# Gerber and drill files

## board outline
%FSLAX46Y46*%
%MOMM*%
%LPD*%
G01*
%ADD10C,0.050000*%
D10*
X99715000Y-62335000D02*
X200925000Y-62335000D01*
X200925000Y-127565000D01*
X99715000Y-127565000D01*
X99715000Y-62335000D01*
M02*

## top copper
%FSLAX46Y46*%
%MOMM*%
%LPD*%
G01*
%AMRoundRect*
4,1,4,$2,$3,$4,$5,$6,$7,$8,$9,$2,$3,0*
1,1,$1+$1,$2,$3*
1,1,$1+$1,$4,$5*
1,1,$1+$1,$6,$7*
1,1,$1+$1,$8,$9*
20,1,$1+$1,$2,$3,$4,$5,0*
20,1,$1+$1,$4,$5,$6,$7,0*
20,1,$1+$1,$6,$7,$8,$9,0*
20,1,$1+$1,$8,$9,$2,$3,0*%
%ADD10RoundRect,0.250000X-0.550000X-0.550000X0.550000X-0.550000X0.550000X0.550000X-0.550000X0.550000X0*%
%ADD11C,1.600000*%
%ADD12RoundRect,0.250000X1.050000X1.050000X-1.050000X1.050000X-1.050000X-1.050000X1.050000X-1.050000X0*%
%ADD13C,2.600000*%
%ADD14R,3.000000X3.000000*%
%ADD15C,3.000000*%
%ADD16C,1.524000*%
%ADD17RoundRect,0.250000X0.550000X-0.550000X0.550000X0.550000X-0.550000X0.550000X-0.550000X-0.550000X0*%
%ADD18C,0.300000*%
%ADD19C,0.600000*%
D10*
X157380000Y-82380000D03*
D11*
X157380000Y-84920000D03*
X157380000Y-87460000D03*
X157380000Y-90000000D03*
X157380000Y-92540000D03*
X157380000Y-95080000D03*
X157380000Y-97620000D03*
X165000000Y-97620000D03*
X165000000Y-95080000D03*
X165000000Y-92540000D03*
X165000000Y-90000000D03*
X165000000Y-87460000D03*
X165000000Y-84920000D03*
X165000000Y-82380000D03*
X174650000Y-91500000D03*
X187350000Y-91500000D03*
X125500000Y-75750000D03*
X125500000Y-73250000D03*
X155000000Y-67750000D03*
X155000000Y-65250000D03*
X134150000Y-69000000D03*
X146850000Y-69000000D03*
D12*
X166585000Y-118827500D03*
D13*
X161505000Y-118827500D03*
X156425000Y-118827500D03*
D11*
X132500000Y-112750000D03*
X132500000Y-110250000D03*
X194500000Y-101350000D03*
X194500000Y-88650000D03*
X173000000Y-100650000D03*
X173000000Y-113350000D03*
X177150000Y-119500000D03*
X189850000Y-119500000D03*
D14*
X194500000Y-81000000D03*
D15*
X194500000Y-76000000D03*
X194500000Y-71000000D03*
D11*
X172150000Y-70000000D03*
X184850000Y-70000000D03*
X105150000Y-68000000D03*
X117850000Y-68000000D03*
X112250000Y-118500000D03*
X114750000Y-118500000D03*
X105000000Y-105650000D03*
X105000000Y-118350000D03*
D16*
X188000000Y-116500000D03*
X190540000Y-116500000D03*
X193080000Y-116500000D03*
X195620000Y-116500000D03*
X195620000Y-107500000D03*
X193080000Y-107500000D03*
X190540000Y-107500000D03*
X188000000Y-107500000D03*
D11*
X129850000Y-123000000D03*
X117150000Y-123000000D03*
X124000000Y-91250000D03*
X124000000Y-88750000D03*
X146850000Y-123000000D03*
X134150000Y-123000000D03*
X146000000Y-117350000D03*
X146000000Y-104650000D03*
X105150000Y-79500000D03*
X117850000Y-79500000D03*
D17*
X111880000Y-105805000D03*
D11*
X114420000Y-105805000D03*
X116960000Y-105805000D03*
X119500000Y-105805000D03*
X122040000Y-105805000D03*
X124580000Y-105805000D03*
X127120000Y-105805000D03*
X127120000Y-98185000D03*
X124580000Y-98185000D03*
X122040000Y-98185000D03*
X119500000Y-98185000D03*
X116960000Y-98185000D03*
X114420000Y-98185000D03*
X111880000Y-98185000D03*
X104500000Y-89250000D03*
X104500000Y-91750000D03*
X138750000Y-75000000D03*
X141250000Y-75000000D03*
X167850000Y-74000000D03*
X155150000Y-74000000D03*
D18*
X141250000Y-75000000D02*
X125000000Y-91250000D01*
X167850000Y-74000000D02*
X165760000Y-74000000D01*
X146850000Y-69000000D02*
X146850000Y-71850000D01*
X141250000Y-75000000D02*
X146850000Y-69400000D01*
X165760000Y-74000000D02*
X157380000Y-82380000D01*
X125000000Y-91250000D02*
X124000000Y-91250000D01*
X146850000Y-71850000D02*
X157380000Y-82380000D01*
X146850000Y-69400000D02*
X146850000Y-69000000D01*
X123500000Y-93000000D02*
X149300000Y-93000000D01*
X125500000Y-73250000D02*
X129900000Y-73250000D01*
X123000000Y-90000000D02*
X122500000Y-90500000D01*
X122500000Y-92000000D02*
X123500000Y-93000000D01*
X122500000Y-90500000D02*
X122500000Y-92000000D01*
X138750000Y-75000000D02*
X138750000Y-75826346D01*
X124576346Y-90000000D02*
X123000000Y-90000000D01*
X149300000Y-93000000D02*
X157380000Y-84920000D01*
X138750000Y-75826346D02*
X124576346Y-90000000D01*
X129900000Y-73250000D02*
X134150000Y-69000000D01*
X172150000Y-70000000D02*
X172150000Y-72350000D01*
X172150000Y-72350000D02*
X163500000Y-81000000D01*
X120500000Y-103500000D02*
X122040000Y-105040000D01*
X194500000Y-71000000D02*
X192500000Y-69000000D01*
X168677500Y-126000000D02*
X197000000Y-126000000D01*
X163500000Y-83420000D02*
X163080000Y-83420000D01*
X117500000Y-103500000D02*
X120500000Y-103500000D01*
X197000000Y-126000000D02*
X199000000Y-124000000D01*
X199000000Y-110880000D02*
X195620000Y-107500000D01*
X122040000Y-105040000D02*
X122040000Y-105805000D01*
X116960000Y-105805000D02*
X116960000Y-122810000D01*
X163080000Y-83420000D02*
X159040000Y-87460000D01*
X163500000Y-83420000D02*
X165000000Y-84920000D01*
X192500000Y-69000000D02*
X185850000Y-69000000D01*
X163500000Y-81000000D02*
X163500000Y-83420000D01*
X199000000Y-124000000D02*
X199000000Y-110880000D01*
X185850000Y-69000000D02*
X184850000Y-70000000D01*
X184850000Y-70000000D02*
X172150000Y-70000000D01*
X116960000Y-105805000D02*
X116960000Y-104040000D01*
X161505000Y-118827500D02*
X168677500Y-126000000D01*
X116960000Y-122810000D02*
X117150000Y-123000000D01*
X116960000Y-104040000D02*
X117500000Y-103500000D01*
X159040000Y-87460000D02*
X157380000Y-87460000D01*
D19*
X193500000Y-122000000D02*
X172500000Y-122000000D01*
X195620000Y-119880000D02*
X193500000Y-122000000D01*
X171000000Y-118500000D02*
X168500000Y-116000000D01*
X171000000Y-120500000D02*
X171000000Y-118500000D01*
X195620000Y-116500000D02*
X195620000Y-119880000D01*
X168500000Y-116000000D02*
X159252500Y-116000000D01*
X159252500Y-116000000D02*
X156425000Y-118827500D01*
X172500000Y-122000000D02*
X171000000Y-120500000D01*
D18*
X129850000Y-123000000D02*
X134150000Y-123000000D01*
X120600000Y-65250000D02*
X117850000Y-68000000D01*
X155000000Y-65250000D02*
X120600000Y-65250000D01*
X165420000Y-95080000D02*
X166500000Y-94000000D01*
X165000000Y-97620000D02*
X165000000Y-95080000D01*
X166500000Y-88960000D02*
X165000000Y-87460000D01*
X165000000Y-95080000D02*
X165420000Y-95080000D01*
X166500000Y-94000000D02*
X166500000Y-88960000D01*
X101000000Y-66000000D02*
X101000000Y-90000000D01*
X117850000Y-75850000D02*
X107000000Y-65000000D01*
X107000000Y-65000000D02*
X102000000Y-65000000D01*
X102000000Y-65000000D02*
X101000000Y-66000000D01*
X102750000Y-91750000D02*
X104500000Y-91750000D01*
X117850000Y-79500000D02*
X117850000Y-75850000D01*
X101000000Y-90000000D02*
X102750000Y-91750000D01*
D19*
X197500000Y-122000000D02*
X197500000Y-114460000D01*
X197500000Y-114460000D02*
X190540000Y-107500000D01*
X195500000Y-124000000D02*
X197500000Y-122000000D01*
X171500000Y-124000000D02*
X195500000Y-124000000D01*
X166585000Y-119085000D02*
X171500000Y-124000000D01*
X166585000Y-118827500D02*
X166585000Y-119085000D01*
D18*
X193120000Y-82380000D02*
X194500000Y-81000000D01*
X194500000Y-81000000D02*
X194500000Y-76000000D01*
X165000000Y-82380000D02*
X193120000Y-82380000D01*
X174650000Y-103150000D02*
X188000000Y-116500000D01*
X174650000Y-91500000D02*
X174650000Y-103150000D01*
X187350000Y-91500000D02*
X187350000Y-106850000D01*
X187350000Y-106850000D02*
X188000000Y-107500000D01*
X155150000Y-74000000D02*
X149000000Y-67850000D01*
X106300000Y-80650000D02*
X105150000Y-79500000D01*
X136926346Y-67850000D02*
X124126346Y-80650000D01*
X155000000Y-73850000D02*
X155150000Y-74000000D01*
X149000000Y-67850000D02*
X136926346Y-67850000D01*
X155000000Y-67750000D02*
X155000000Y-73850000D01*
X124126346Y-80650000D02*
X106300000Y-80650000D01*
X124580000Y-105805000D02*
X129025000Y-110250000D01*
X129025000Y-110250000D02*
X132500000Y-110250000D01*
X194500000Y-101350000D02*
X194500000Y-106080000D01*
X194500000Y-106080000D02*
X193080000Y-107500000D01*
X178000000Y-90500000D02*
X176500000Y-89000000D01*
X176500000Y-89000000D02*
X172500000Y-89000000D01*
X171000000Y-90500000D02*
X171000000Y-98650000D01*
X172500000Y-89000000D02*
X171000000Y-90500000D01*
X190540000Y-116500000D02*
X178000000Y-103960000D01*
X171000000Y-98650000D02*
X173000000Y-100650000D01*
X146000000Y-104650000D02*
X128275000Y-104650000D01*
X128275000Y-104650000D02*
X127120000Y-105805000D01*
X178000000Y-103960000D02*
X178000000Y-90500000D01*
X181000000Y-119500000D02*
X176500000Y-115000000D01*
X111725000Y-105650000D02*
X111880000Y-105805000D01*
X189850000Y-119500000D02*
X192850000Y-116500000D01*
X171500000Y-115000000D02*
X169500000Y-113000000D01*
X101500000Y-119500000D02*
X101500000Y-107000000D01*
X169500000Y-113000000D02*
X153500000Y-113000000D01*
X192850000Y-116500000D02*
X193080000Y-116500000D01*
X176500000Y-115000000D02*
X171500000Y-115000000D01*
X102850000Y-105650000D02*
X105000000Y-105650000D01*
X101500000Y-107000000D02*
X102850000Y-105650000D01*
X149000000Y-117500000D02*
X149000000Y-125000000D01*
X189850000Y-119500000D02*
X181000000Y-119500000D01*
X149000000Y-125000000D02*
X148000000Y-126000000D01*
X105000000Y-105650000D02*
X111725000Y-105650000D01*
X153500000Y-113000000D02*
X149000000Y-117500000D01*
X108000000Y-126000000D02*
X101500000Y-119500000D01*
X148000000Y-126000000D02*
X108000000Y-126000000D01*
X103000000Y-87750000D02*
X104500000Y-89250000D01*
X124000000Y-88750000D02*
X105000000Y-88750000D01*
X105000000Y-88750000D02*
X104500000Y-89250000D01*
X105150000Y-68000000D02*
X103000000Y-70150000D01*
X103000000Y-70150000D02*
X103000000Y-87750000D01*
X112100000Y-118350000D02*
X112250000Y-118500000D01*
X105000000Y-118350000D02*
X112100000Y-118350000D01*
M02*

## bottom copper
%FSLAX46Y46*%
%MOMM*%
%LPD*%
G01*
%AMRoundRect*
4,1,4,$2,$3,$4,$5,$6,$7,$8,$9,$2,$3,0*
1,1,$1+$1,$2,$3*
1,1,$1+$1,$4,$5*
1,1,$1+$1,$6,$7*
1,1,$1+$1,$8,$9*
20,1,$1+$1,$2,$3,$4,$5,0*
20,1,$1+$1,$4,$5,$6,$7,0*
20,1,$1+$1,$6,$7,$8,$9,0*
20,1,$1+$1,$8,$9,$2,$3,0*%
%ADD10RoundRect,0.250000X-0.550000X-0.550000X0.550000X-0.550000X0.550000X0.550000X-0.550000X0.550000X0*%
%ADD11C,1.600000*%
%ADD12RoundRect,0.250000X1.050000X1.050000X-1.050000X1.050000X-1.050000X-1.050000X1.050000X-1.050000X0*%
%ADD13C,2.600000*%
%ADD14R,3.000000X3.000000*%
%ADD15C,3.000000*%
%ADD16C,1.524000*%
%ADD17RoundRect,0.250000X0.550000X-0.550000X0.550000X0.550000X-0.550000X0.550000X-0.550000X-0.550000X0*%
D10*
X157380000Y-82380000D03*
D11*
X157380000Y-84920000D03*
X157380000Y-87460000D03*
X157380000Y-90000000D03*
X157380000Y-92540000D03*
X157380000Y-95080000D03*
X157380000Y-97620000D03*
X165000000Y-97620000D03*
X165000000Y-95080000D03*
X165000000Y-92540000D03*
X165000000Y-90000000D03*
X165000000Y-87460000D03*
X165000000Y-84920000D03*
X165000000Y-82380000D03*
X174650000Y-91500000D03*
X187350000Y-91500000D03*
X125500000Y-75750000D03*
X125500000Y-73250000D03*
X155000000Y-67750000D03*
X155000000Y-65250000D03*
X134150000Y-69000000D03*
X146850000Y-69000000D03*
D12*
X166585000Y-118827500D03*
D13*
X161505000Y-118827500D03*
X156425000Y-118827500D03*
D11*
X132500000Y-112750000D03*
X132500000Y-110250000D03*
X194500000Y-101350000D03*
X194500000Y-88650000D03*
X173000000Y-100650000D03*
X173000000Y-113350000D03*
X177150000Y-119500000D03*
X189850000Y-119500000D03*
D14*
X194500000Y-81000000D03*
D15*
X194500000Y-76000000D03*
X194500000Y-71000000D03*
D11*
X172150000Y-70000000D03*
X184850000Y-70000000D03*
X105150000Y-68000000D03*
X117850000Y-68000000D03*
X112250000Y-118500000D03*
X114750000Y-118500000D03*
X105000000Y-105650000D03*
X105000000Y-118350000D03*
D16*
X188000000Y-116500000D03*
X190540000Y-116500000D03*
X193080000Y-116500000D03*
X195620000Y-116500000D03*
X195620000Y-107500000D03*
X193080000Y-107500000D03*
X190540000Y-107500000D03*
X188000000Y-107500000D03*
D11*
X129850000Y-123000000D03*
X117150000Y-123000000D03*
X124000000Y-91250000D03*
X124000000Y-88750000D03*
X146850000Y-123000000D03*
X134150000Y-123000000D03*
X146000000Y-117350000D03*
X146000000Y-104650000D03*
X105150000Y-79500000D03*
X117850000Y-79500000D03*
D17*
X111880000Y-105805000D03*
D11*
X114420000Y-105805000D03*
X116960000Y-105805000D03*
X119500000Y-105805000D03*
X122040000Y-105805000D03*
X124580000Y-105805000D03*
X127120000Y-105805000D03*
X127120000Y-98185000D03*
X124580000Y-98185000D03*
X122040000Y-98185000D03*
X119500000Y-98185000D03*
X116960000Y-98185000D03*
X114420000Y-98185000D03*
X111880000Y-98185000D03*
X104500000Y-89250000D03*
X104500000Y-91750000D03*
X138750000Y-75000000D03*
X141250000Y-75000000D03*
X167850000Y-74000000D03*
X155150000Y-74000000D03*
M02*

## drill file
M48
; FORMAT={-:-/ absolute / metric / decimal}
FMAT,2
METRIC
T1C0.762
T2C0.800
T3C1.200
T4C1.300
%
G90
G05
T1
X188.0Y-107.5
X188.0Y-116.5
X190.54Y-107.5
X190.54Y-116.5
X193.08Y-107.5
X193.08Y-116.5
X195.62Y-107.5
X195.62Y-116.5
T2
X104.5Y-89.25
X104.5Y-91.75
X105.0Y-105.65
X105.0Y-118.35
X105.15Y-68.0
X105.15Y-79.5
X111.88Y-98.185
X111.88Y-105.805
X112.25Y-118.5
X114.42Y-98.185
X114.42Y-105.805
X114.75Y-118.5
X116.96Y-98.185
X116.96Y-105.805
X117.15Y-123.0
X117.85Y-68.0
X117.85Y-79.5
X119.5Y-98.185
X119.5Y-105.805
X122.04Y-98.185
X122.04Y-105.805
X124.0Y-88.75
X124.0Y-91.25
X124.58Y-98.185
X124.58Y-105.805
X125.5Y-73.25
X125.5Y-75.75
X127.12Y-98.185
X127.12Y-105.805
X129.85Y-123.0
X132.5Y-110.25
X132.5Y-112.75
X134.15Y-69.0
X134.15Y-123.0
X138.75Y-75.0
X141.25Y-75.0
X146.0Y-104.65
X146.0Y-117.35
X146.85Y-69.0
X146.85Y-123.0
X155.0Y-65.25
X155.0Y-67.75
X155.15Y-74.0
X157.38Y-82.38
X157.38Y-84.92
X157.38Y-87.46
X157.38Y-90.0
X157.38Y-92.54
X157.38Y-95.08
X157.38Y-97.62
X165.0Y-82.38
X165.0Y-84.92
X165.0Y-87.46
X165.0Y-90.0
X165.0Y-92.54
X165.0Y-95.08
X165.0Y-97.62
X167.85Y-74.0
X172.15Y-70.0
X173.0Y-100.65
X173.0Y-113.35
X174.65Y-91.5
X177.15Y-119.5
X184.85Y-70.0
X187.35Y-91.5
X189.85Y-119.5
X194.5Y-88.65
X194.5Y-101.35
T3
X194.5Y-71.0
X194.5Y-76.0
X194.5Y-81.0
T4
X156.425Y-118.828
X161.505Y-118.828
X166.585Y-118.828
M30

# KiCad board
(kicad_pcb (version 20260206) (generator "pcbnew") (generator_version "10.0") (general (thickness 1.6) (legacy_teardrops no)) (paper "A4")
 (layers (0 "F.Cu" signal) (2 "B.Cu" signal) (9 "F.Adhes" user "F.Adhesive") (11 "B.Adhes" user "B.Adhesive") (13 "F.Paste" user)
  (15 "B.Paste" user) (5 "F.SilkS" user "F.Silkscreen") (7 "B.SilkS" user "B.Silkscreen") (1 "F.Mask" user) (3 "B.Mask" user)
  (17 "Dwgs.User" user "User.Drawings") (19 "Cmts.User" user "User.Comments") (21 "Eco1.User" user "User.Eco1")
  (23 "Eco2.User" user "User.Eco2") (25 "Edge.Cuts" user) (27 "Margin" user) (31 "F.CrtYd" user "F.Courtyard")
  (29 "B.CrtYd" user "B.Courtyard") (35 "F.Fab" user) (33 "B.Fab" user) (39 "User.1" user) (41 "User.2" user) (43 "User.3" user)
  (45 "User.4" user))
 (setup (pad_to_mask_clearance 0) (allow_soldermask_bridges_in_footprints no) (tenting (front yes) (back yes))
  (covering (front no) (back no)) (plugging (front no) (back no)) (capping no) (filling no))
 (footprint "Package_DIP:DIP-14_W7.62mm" (layer "F.Cu") (at 157.38 82.38)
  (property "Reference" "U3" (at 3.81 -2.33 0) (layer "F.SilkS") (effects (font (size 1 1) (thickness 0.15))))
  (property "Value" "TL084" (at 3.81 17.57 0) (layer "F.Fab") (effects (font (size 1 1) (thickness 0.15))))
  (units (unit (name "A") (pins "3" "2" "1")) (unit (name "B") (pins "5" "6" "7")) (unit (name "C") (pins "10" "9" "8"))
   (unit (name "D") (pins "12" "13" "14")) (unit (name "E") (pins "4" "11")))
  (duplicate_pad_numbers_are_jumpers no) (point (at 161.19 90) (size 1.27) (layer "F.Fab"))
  (pad "1" thru_hole roundrect (at 0 0) (size 1.6 1.6) (drill 0.8) (layers "*.Cu" "*.Mask") (remove_unused_layers no)
   (roundrect_rratio 0.15625) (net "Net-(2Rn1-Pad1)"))
  (pad "2" thru_hole circle (at 0 2.54) (size 1.6 1.6) (drill 0.8) (layers "*.Cu" "*.Mask") (remove_unused_layers no) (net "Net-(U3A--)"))
  (pad "3" thru_hole circle (at 0 5.08) (size 1.6 1.6) (drill 0.8) (layers "*.Cu" "*.Mask") (remove_unused_layers no) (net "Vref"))
  (pad "4" thru_hole circle (at 0 7.62) (size 1.6 1.6) (drill 0.8) (layers "*.Cu" "*.Mask") (remove_unused_layers no) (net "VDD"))
  (pad "5" thru_hole circle (at 0 10.16) (size 1.6 1.6) (drill 0.8) (layers "*.Cu" "*.Mask") (remove_unused_layers no) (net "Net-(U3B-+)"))
  (pad "6" thru_hole circle (at 0 12.7) (size 1.6 1.6) (drill 0.8) (layers "*.Cu" "*.Mask") (remove_unused_layers no) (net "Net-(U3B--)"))
  (pad "7" thru_hole circle (at 0 15.24) (size 1.6 1.6) (drill 0.8) (layers "*.Cu" "*.Mask") (remove_unused_layers no) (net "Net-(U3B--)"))
  (pad "8" thru_hole circle (at 7.62 15.24) (size 1.6 1.6) (drill 0.8) (layers "*.Cu" "*.Mask") (remove_unused_layers no)
   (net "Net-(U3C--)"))
  (pad "9" thru_hole circle (at 7.62 12.7) (size 1.6 1.6) (drill 0.8) (layers "*.Cu" "*.Mask") (remove_unused_layers no) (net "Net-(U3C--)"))
  (pad "10" thru_hole circle (at 7.62 10.16) (size 1.6 1.6) (drill 0.8) (layers "*.Cu" "*.Mask") (remove_unused_layers no)
   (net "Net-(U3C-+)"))
  (pad "11" thru_hole circle (at 7.62 7.62) (size 1.6 1.6) (drill 0.8) (layers "*.Cu" "*.Mask") (remove_unused_layers no) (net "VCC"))
  (pad "12" thru_hole circle (at 7.62 5.08) (size 1.6 1.6) (drill 0.8) (layers "*.Cu" "*.Mask") (remove_unused_layers no)
   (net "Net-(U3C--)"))
  (pad "13" thru_hole circle (at 7.62 2.54) (size 1.6 1.6) (drill 0.8) (layers "*.Cu" "*.Mask") (remove_unused_layers no) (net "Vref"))
  (pad "14" thru_hole circle (at 7.62 0) (size 1.6 1.6) (drill 0.8) (layers "*.Cu" "*.Mask") (remove_unused_layers no) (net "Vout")))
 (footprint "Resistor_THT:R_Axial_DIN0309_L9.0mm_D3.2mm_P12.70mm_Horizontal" (layer "F.Cu") (at 174.65 91.5)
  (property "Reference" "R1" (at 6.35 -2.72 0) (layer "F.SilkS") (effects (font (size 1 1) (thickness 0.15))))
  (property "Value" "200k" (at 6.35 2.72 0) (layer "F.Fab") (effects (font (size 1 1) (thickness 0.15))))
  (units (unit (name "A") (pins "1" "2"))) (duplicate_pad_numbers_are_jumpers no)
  (pad "1" thru_hole circle (at 0 0) (size 1.6 1.6) (drill 0.8) (layers "*.Cu" "*.Mask") (remove_unused_layers no) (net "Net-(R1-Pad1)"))
  (pad "2" thru_hole circle (at 12.7 0) (size 1.6 1.6) (drill 0.8) (layers "*.Cu" "*.Mask") (remove_unused_layers no) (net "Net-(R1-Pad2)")))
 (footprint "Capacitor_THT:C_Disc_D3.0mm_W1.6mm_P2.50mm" (layer "F.Cu") (at 125.5 75.75 90)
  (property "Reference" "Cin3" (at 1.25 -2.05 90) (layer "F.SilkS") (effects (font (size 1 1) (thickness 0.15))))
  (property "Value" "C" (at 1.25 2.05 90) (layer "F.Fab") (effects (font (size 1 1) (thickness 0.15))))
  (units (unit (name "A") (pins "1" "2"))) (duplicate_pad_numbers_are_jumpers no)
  (pad "1" thru_hole circle (at 0 0 90) (size 1.6 1.6) (drill 0.8) (layers "*.Cu" "*.Mask") (remove_unused_layers no)
   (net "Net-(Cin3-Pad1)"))
  (pad "2" thru_hole circle (at 2.5 0 90) (size 1.6 1.6) (drill 0.8) (layers "*.Cu" "*.Mask") (remove_unused_layers no) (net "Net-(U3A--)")))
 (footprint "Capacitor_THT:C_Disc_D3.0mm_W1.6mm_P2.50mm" (layer "F.Cu") (at 155 67.75 90)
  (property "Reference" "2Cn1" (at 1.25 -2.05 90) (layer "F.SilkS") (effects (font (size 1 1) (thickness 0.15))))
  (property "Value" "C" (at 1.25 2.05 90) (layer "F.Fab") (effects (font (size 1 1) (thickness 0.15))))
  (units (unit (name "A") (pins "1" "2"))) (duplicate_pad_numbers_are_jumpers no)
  (pad "1" thru_hole circle (at 0 0 90) (size 1.6 1.6) (drill 0.8) (layers "*.Cu" "*.Mask") (remove_unused_layers no)
   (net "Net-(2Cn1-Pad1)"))
  (pad "2" thru_hole circle (at 2.5 0 90) (size 1.6 1.6) (drill 0.8) (layers "*.Cu" "*.Mask") (remove_unused_layers no) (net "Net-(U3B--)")))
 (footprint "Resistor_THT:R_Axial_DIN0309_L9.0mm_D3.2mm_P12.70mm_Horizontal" (layer "F.Cu") (at 134.15 69)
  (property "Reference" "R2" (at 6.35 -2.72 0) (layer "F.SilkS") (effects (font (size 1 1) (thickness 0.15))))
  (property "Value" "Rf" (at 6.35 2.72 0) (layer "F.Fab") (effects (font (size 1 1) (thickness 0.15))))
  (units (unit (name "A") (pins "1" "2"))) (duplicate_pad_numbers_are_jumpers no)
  (pad "1" thru_hole circle (at 0 0) (size 1.6 1.6) (drill 0.8) (layers "*.Cu" "*.Mask") (remove_unused_layers no) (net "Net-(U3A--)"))
  (pad "2" thru_hole circle (at 12.7 0) (size 1.6 1.6) (drill 0.8) (layers "*.Cu" "*.Mask") (remove_unused_layers no)
   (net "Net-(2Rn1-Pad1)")))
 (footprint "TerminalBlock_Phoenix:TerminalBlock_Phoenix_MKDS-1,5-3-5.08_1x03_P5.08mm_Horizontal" (layer "F.Cu") (at 166.585 118.8275 180)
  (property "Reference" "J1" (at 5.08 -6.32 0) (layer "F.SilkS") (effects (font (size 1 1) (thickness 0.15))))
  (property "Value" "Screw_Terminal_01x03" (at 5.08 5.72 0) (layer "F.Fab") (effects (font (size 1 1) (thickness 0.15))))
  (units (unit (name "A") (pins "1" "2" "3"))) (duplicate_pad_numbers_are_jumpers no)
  (pad "1" thru_hole roundrect (at 0 0 180) (size 2.6 2.6) (drill 1.3) (layers "*.Cu" "*.Mask") (remove_unused_layers no)
   (roundrect_rratio 0.096154) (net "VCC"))
  (pad "2" thru_hole circle (at 5.08 0 180) (size 2.6 2.6) (drill 1.3) (layers "*.Cu" "*.Mask") (remove_unused_layers no) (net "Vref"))
  (pad "3" thru_hole circle (at 10.16 0 180) (size 2.6 2.6) (drill 1.3) (layers "*.Cu" "*.Mask") (remove_unused_layers no) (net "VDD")))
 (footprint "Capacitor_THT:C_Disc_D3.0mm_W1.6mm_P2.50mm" (layer "F.Cu") (at 132.5 112.75 90)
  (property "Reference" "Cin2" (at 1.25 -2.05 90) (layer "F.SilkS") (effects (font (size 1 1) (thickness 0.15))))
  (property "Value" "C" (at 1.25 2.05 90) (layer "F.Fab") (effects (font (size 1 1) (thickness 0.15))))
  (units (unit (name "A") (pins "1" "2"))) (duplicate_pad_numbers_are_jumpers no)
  (pad "1" thru_hole circle (at 0 0 90) (size 1.6 1.6) (drill 0.8) (layers "*.Cu" "*.Mask") (remove_unused_layers no)
   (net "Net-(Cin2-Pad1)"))
  (pad "2" thru_hole circle (at 2.5 0 90) (size 1.6 1.6) (drill 0.8) (layers "*.Cu" "*.Mask") (remove_unused_layers no) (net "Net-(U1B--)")))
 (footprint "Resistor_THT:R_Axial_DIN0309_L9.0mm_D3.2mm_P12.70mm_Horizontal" (layer "F.Cu") (at 194.5 101.35 90)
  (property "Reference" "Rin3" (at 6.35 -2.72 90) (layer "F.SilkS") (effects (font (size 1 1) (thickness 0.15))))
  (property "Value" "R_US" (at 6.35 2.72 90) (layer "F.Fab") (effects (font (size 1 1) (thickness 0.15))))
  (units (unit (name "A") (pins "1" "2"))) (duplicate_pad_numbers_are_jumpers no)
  (pad "1" thru_hole circle (at 0 0 90) (size 1.6 1.6) (drill 0.8) (layers "*.Cu" "*.Mask") (remove_unused_layers no) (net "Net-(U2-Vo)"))
  (pad "2" thru_hole circle (at 12.7 0 90) (size 1.6 1.6) (drill 0.8) (layers "*.Cu" "*.Mask") (remove_unused_layers no)
   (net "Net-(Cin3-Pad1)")))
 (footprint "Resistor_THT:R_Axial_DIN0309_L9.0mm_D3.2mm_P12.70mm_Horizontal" (layer "F.Cu") (at 173 100.65 -90)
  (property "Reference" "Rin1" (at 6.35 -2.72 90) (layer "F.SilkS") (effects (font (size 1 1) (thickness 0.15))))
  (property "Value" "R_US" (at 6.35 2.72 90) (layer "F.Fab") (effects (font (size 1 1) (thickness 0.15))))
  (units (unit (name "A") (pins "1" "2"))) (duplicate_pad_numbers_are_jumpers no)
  (pad "1" thru_hole circle (at 0 0 270) (size 1.6 1.6) (drill 0.8) (layers "*.Cu" "*.Mask") (remove_unused_layers no) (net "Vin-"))
  (pad "2" thru_hole circle (at 12.7 0 270) (size 1.6 1.6) (drill 0.8) (layers "*.Cu" "*.Mask") (remove_unused_layers no)
   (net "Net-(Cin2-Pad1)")))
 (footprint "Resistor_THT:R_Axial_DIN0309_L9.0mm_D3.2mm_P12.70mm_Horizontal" (layer "F.Cu") (at 177.15 119.5)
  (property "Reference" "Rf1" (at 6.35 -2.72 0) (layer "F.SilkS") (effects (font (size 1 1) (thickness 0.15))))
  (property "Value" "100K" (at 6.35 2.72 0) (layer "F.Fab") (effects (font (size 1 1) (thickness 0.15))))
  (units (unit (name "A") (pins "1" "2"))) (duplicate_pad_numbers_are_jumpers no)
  (pad "1" thru_hole circle (at 0 0) (size 1.6 1.6) (drill 0.8) (layers "*.Cu" "*.Mask") (remove_unused_layers no) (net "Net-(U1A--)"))
  (pad "2" thru_hole circle (at 12.7 0) (size 1.6 1.6) (drill 0.8) (layers "*.Cu" "*.Mask") (remove_unused_layers no) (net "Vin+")))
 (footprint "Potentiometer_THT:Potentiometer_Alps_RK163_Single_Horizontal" (layer "F.Cu") (at 194.5 81 180)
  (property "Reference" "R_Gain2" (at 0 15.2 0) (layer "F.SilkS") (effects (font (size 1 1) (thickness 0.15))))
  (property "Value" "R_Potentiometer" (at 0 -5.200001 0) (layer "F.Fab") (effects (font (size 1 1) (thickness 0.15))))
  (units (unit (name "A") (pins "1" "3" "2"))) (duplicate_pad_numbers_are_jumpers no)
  (pad "1" thru_hole rect (at 0 0) (size 3 3) (drill 1.2) (layers "*.Cu" "*.Mask") (remove_unused_layers no) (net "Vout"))
  (pad "2" thru_hole circle (at 0 5) (size 3 3) (drill 1.2) (layers "*.Cu" "*.Mask") (remove_unused_layers no) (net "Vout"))
  (pad "3" thru_hole circle (at 0 10) (size 3 3) (drill 1.2) (layers "*.Cu" "*.Mask") (remove_unused_layers no) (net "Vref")))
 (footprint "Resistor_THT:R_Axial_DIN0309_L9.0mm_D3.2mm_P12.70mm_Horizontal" (layer "F.Cu") (at 172.15 70)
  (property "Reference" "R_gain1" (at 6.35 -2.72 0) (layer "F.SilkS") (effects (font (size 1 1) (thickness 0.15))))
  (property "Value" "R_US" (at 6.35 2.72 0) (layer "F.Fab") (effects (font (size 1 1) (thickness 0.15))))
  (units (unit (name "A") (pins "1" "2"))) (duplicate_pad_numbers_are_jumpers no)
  (pad "1" thru_hole circle (at 0 0) (size 1.6 1.6) (drill 0.8) (layers "*.Cu" "*.Mask") (remove_unused_layers no) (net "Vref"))
  (pad "2" thru_hole circle (at 12.7 0) (size 1.6 1.6) (drill 0.8) (layers "*.Cu" "*.Mask") (remove_unused_layers no) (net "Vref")))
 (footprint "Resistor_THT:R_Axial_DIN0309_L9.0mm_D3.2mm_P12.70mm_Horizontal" (layer "F.Cu") (at 105.15 68)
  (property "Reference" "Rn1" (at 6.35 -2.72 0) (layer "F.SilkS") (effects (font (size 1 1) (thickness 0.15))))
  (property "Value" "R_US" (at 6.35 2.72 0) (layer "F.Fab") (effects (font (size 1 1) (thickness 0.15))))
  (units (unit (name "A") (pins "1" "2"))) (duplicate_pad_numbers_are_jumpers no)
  (pad "1" thru_hole circle (at 0 0) (size 1.6 1.6) (drill 0.8) (layers "*.Cu" "*.Mask") (remove_unused_layers no) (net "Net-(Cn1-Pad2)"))
  (pad "2" thru_hole circle (at 12.7 0) (size 1.6 1.6) (drill 0.8) (layers "*.Cu" "*.Mask") (remove_unused_layers no) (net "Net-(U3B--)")))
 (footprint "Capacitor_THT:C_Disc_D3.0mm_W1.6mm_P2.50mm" (layer "F.Cu") (at 112.25 118.5)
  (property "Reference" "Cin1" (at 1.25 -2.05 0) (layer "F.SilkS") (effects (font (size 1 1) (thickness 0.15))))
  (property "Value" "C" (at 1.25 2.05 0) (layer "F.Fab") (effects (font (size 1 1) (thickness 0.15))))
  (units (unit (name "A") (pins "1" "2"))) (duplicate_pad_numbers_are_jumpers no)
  (pad "1" thru_hole circle (at 0 0) (size 1.6 1.6) (drill 0.8) (layers "*.Cu" "*.Mask") (remove_unused_layers no) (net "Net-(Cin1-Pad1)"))
  (pad "2" thru_hole circle (at 2.5 0) (size 1.6 1.6) (drill 0.8) (layers "*.Cu" "*.Mask") (remove_unused_layers no) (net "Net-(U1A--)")))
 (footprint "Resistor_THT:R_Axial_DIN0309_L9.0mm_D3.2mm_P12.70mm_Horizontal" (layer "F.Cu") (at 105 105.65 -90)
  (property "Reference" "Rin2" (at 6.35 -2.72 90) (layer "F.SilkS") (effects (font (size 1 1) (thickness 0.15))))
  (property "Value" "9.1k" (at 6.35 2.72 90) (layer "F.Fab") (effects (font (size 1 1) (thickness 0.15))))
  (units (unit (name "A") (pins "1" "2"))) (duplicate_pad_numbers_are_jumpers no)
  (pad "1" thru_hole circle (at 0 0 270) (size 1.6 1.6) (drill 0.8) (layers "*.Cu" "*.Mask") (remove_unused_layers no) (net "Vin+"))
  (pad "2" thru_hole circle (at 12.7 0 270) (size 1.6 1.6) (drill 0.8) (layers "*.Cu" "*.Mask") (remove_unused_layers no)
   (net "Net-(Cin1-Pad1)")))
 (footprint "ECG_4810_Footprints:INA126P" (layer "F.Cu") (at 192 112 90)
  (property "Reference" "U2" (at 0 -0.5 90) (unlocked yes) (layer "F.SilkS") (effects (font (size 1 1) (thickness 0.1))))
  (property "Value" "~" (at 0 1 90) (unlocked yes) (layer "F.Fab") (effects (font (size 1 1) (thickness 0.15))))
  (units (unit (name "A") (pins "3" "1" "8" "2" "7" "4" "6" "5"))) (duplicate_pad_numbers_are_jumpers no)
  (pad "1" thru_hole circle (at -4.5 -4) (size 1.524 1.524) (drill 0.762) (layers "*.Cu" "*.Mask") (remove_unused_layers no)
   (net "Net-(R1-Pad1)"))
  (pad "2" thru_hole circle (at -4.5 -1.46) (size 1.524 1.524) (drill 0.762) (layers "*.Cu" "*.Mask") (remove_unused_layers no) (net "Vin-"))
  (pad "3" thru_hole circle (at -4.5 1.08) (size 1.524 1.524) (drill 0.762) (layers "*.Cu" "*.Mask") (remove_unused_layers no) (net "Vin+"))
  (pad "4" thru_hole circle (at -4.5 3.62) (size 1.524 1.524) (drill 0.762) (layers "*.Cu" "*.Mask") (remove_unused_layers no) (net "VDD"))
  (pad "5" thru_hole circle (at 4.5 3.62 180) (size 1.524 1.524) (drill 0.762) (layers "*.Cu" "*.Mask") (remove_unused_layers no)
   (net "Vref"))
  (pad "6" thru_hole circle (at 4.5 1.08 180) (size 1.524 1.524) (drill 0.762) (layers "*.Cu" "*.Mask") (remove_unused_layers no)
   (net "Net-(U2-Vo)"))
  (pad "7" thru_hole circle (at 4.5 -1.46 180) (size 1.524 1.524) (drill 0.762) (layers "*.Cu" "*.Mask") (remove_unused_layers no)
   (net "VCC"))
  (pad "8" thru_hole circle (at 4.5 -4 180) (size 1.524 1.524) (drill 0.762) (layers "*.Cu" "*.Mask") (remove_unused_layers no)
   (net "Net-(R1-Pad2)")))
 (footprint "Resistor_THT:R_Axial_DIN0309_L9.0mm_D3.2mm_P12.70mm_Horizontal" (layer "F.Cu") (at 129.85 123 180)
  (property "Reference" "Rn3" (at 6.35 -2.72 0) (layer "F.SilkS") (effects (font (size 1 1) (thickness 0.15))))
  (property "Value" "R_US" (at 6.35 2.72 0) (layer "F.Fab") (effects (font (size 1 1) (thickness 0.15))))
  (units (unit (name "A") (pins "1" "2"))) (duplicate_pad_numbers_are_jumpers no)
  (pad "1" thru_hole circle (at 0 0 180) (size 1.6 1.6) (drill 0.8) (layers "*.Cu" "*.Mask") (remove_unused_layers no) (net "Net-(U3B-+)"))
  (pad "2" thru_hole circle (at 12.7 0 180) (size 1.6 1.6) (drill 0.8) (layers "*.Cu" "*.Mask") (remove_unused_layers no) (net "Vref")))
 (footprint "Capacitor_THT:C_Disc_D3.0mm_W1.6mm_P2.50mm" (layer "F.Cu") (at 124 91.25 90)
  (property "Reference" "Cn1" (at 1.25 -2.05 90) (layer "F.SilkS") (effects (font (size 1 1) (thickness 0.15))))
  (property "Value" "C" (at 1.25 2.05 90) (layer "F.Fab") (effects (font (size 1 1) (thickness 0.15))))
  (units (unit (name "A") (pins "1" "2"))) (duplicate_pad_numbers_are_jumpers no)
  (pad "1" thru_hole circle (at 0 0 90) (size 1.6 1.6) (drill 0.8) (layers "*.Cu" "*.Mask") (remove_unused_layers no)
   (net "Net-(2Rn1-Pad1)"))
  (pad "2" thru_hole circle (at 2.5 0 90) (size 1.6 1.6) (drill 0.8) (layers "*.Cu" "*.Mask") (remove_unused_layers no)
   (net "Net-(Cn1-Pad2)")))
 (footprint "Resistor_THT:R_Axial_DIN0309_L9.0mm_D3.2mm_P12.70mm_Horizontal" (layer "F.Cu") (at 146.85 123 180)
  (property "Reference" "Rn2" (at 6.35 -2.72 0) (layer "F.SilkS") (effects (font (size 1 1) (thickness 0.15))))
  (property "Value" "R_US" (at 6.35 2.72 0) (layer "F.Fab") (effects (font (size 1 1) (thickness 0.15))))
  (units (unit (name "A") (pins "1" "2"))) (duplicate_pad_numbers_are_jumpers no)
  (pad "1" thru_hole circle (at 0 0 180) (size 1.6 1.6) (drill 0.8) (layers "*.Cu" "*.Mask") (remove_unused_layers no) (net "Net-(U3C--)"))
  (pad "2" thru_hole circle (at 12.7 0 180) (size 1.6 1.6) (drill 0.8) (layers "*.Cu" "*.Mask") (remove_unused_layers no)
   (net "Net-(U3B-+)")))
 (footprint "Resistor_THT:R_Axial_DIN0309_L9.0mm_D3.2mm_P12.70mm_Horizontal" (layer "F.Cu") (at 146 117.35 90)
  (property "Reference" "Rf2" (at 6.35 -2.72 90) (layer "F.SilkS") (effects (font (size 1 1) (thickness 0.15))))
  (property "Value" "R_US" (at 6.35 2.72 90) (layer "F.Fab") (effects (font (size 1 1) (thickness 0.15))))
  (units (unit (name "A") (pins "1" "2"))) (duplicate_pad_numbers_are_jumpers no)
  (pad "1" thru_hole circle (at 0 0 90) (size 1.6 1.6) (drill 0.8) (layers "*.Cu" "*.Mask") (remove_unused_layers no) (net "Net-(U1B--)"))
  (pad "2" thru_hole circle (at 12.7 0 90) (size 1.6 1.6) (drill 0.8) (layers "*.Cu" "*.Mask") (remove_unused_layers no) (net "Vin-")))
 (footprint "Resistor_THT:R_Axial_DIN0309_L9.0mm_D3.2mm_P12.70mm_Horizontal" (layer "F.Cu") (at 105.15 79.5)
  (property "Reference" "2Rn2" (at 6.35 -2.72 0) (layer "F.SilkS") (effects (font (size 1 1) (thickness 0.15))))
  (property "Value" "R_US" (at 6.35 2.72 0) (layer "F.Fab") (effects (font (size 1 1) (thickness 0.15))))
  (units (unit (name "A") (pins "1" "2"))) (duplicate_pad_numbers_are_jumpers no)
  (pad "1" thru_hole circle (at 0 0) (size 1.6 1.6) (drill 0.8) (layers "*.Cu" "*.Mask") (remove_unused_layers no) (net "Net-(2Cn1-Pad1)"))
  (pad "2" thru_hole circle (at 12.7 0) (size 1.6 1.6) (drill 0.8) (layers "*.Cu" "*.Mask") (remove_unused_layers no) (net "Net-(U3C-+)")))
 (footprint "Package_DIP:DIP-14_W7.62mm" (layer "F.Cu") (at 111.88 105.805 90)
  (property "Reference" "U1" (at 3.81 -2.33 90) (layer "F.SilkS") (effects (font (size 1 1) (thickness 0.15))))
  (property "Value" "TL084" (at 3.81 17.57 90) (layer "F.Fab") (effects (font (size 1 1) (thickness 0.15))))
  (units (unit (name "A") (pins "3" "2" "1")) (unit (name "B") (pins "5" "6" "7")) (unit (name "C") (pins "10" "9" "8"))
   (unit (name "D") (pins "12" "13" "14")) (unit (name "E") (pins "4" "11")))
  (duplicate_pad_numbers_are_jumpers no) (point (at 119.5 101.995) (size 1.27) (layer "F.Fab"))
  (pad "1" thru_hole roundrect (at 0 0 90) (size 1.6 1.6) (drill 0.8) (layers "*.Cu" "*.Mask") (remove_unused_layers no)
   (roundrect_rratio 0.15625) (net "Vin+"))
  (pad "2" thru_hole circle (at 0 2.54 90) (size 1.6 1.6) (drill 0.8) (layers "*.Cu" "*.Mask") (remove_unused_layers no) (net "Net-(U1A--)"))
  (pad "3" thru_hole circle (at 0 5.08 90) (size 1.6 1.6) (drill 0.8) (layers "*.Cu" "*.Mask") (remove_unused_layers no) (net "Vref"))
  (pad "4" thru_hole circle (at 0 7.62 90) (size 1.6 1.6) (drill 0.8) (layers "*.Cu" "*.Mask") (remove_unused_layers no) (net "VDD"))
  (pad "5" thru_hole circle (at 0 10.16 90) (size 1.6 1.6) (drill 0.8) (layers "*.Cu" "*.Mask") (remove_unused_layers no) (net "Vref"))
  (pad "6" thru_hole circle (at 0 12.7 90) (size 1.6 1.6) (drill 0.8) (layers "*.Cu" "*.Mask") (remove_unused_layers no) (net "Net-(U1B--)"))
  (pad "7" thru_hole circle (at 0 15.24 90) (size 1.6 1.6) (drill 0.8) (layers "*.Cu" "*.Mask") (remove_unused_layers no) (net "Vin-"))
  (pad "8" thru_hole circle (at 7.62 15.24 90) (size 1.6 1.6) (drill 0.8) (layers "*.Cu" "*.Mask") (remove_unused_layers no))
  (pad "9" thru_hole circle (at 7.62 12.7 90) (size 1.6 1.6) (drill 0.8) (layers "*.Cu" "*.Mask") (remove_unused_layers no))
  (pad "10" thru_hole circle (at 7.62 10.16 90) (size 1.6 1.6) (drill 0.8) (layers "*.Cu" "*.Mask") (remove_unused_layers no))
  (pad "11" thru_hole circle (at 7.62 7.62 90) (size 1.6 1.6) (drill 0.8) (layers "*.Cu" "*.Mask") (remove_unused_layers no) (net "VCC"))
  (pad "12" thru_hole circle (at 7.62 5.08 90) (size 1.6 1.6) (drill 0.8) (layers "*.Cu" "*.Mask") (remove_unused_layers no))
  (pad "13" thru_hole circle (at 7.62 2.54 90) (size 1.6 1.6) (drill 0.8) (layers "*.Cu" "*.Mask") (remove_unused_layers no))
  (pad "14" thru_hole circle (at 7.62 0 90) (size 1.6 1.6) (drill 0.8) (layers "*.Cu" "*.Mask") (remove_unused_layers no)))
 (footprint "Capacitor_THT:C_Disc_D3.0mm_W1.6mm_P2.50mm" (layer "F.Cu") (at 104.5 89.25 -90)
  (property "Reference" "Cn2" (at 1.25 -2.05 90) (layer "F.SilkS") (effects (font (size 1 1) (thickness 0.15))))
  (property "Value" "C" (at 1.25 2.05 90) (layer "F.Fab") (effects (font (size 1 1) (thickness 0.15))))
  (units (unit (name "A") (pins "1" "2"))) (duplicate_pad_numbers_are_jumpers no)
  (pad "1" thru_hole circle (at 0 0 270) (size 1.6 1.6) (drill 0.8) (layers "*.Cu" "*.Mask") (remove_unused_layers no)
   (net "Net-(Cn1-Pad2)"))
  (pad "2" thru_hole circle (at 2.5 0 270) (size 1.6 1.6) (drill 0.8) (layers "*.Cu" "*.Mask") (remove_unused_layers no) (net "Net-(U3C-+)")))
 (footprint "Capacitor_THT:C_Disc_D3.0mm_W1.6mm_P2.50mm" (layer "F.Cu") (at 138.75 75)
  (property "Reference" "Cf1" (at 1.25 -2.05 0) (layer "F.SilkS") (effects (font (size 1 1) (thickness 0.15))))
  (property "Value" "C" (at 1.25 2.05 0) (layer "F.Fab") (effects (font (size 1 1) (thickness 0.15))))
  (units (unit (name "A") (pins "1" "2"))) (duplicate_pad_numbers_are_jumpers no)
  (pad "1" thru_hole circle (at 0 0) (size 1.6 1.6) (drill 0.8) (layers "*.Cu" "*.Mask") (remove_unused_layers no) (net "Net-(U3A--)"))
  (pad "2" thru_hole circle (at 2.5 0) (size 1.6 1.6) (drill 0.8) (layers "*.Cu" "*.Mask") (remove_unused_layers no) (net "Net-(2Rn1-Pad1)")))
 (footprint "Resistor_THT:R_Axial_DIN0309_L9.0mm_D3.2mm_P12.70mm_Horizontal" (layer "F.Cu") (at 167.85 74 180)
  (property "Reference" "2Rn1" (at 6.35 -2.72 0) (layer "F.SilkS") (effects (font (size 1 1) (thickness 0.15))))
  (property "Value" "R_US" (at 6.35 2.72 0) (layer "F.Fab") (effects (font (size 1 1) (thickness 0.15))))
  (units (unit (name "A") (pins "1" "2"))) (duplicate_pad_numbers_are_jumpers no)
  (pad "1" thru_hole circle (at 0 0 180) (size 1.6 1.6) (drill 0.8) (layers "*.Cu" "*.Mask") (remove_unused_layers no)
   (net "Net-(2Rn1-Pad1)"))
  (pad "2" thru_hole circle (at 12.7 0 180) (size 1.6 1.6) (drill 0.8) (layers "*.Cu" "*.Mask") (remove_unused_layers no)
   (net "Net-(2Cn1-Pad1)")))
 (gr_rect (start 99.715 62.335) (end 200.925 127.565) (stroke (width 0.05) (type solid)) (fill no) (layer "Edge.Cuts"))
 (segment (start 141.25 75) (end 125 91.25) (width 0.3) (layer "F.Cu") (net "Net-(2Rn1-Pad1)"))
 (segment (start 167.85 74) (end 165.76 74) (width 0.3) (layer "F.Cu") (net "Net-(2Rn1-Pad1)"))
 (segment (start 146.85 69) (end 146.85 71.85) (width 0.3) (layer "F.Cu") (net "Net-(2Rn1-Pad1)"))
 (segment (start 141.25 75) (end 146.85 69.4) (width 0.3) (layer "F.Cu") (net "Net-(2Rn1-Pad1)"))
 (segment (start 165.76 74) (end 157.38 82.38) (width 0.3) (layer "F.Cu") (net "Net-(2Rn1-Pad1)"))
 (segment (start 125 91.25) (end 124 91.25) (width 0.3) (layer "F.Cu") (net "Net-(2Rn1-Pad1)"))
 (segment (start 146.85 71.85) (end 157.38 82.38) (width 0.3) (layer "F.Cu") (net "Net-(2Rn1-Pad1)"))
 (segment (start 146.85 69.4) (end 146.85 69) (width 0.3) (layer "F.Cu") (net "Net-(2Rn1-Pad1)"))
 (segment (start 123.5 93) (end 149.3 93) (width 0.3) (layer "F.Cu") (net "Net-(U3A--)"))
 (segment (start 125.5 73.25) (end 129.9 73.25) (width 0.3) (layer "F.Cu") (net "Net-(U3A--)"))
 (segment (start 123 90) (end 122.5 90.5) (width 0.3) (layer "F.Cu") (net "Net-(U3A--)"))
 (segment (start 122.5 92) (end 123.5 93) (width 0.3) (layer "F.Cu") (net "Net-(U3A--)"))
 (segment (start 122.5 90.5) (end 122.5 92) (width 0.3) (layer "F.Cu") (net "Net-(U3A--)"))
 (segment (start 138.75 75) (end 138.75 75.826346) (width 0.3) (layer "F.Cu") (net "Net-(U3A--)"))
 (segment (start 124.576346 90) (end 123 90) (width 0.3) (layer "F.Cu") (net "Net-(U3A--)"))
 (segment (start 149.3 93) (end 157.38 84.92) (width 0.3) (layer "F.Cu") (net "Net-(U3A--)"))
 (segment (start 138.75 75.826346) (end 124.576346 90) (width 0.3) (layer "F.Cu") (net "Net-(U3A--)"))
 (segment (start 129.9 73.25) (end 134.15 69) (width 0.3) (layer "F.Cu") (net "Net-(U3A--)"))
 (segment (start 172.15 70) (end 172.15 72.35) (width 0.3) (layer "F.Cu") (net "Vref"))
 (segment (start 172.15 72.35) (end 163.5 81) (width 0.3) (layer "F.Cu") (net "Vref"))
 (segment (start 120.5 103.5) (end 122.04 105.04) (width 0.3) (layer "F.Cu") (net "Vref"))
 (segment (start 194.5 71) (end 192.5 69) (width 0.3) (layer "F.Cu") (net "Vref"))
 (segment (start 168.6775 126) (end 197 126) (width 0.3) (layer "F.Cu") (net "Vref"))
 (segment (start 163.5 83.42) (end 163.08 83.42) (width 0.3) (layer "F.Cu") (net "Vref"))
 (segment (start 117.5 103.5) (end 120.5 103.5) (width 0.3) (layer "F.Cu") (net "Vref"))
 (segment (start 197 126) (end 199 124) (width 0.3) (layer "F.Cu") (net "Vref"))
 (segment (start 199 110.88) (end 195.62 107.5) (width 0.3) (layer "F.Cu") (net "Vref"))
 (segment (start 122.04 105.04) (end 122.04 105.805) (width 0.3) (layer "F.Cu") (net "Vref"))
 (segment (start 116.96 105.805) (end 116.96 122.81) (width 0.3) (layer "F.Cu") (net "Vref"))
 (segment (start 163.08 83.42) (end 159.04 87.46) (width 0.3) (layer "F.Cu") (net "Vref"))
 (segment (start 163.5 83.42) (end 165 84.92) (width 0.3) (layer "F.Cu") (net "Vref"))
 (segment (start 192.5 69) (end 185.85 69) (width 0.3) (layer "F.Cu") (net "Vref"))
 (segment (start 163.5 81) (end 163.5 83.42) (width 0.3) (layer "F.Cu") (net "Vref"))
 (segment (start 199 124) (end 199 110.88) (width 0.3) (layer "F.Cu") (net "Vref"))
 (segment (start 185.85 69) (end 184.85 70) (width 0.3) (layer "F.Cu") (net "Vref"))
 (segment (start 184.85 70) (end 172.15 70) (width 0.3) (layer "F.Cu") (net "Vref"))
 (segment (start 116.96 105.805) (end 116.96 104.04) (width 0.3) (layer "F.Cu") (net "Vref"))
 (segment (start 161.505 118.8275) (end 168.6775 126) (width 0.3) (layer "F.Cu") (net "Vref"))
 (segment (start 116.96 122.81) (end 117.15 123) (width 0.3) (layer "F.Cu") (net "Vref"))
 (segment (start 116.96 104.04) (end 117.5 103.5) (width 0.3) (layer "F.Cu") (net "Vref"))
 (segment (start 159.04 87.46) (end 157.38 87.46) (width 0.3) (layer "F.Cu") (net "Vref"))
 (segment (start 193.5 122) (end 172.5 122) (width 0.6) (layer "F.Cu") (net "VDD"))
 (segment (start 195.62 119.88) (end 193.5 122) (width 0.6) (layer "F.Cu") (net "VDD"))
 (segment (start 171 118.5) (end 168.5 116) (width 0.6) (layer "F.Cu") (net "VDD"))
 (segment (start 171 120.5) (end 171 118.5) (width 0.6) (layer "F.Cu") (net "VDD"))
 (segment (start 195.62 116.5) (end 195.62 119.88) (width 0.6) (layer "F.Cu") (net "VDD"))
 (segment (start 168.5 116) (end 159.2525 116) (width 0.6) (layer "F.Cu") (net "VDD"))
 (segment (start 159.2525 116) (end 156.425 118.8275) (width 0.6) (layer "F.Cu") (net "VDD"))
 (segment (start 172.5 122) (end 171 120.5) (width 0.6) (layer "F.Cu") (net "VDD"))
 (segment (start 129.85 123) (end 134.15 123) (width 0.3) (layer "F.Cu") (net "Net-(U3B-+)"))
 (segment (start 120.6 65.25) (end 117.85 68) (width 0.3) (layer "F.Cu") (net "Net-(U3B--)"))
 (segment (start 155 65.25) (end 120.6 65.25) (width 0.3) (layer "F.Cu") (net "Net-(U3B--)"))
 (segment (start 165.42 95.08) (end 166.5 94) (width 0.3) (layer "F.Cu") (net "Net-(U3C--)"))
 (segment (start 165 97.62) (end 165 95.08) (width 0.3) (layer "F.Cu") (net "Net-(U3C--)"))
 (segment (start 166.5 88.96) (end 165 87.46) (width 0.3) (layer "F.Cu") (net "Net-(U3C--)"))
 (segment (start 165 95.08) (end 165.42 95.08) (width 0.3) (layer "F.Cu") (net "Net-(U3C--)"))
 (segment (start 166.5 94) (end 166.5 88.96) (width 0.3) (layer "F.Cu") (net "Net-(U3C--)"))
 (segment (start 101 66) (end 101 90) (width 0.3) (layer "F.Cu") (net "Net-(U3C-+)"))
 (segment (start 117.85 75.85) (end 107 65) (width 0.3) (layer "F.Cu") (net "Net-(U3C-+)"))
 (segment (start 107 65) (end 102 65) (width 0.3) (layer "F.Cu") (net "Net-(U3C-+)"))
 (segment (start 102 65) (end 101 66) (width 0.3) (layer "F.Cu") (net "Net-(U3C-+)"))
 (segment (start 102.75 91.75) (end 104.5 91.75) (width 0.3) (layer "F.Cu") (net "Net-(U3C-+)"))
 (segment (start 117.85 79.5) (end 117.85 75.85) (width 0.3) (layer "F.Cu") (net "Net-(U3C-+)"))
 (segment (start 101 90) (end 102.75 91.75) (width 0.3) (layer "F.Cu") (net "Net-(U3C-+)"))
 (segment (start 197.5 122) (end 197.5 114.46) (width 0.6) (layer "F.Cu") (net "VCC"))
 (segment (start 197.5 114.46) (end 190.54 107.5) (width 0.6) (layer "F.Cu") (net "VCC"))
 (segment (start 195.5 124) (end 197.5 122) (width 0.6) (layer "F.Cu") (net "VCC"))
 (segment (start 171.5 124) (end 195.5 124) (width 0.6) (layer "F.Cu") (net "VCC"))
 (segment (start 166.585 119.085) (end 171.5 124) (width 0.6) (layer "F.Cu") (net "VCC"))
 (segment (start 166.585 118.8275) (end 166.585 119.085) (width 0.6) (layer "F.Cu") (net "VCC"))
 (segment (start 193.12 82.38) (end 194.5 81) (width 0.3) (layer "F.Cu") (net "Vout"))
 (segment (start 194.5 81) (end 194.5 76) (width 0.3) (layer "F.Cu") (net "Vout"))
 (segment (start 165 82.38) (end 193.12 82.38) (width 0.3) (layer "F.Cu") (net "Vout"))
 (segment (start 174.65 103.15) (end 188 116.5) (width 0.3) (layer "F.Cu") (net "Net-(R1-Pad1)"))
 (segment (start 174.65 91.5) (end 174.65 103.15) (width 0.3) (layer "F.Cu") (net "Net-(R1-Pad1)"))
 (segment (start 187.35 91.5) (end 187.35 106.85) (width 0.3) (layer "F.Cu") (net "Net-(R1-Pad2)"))
 (segment (start 187.35 106.85) (end 188 107.5) (width 0.3) (layer "F.Cu") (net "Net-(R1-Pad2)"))
 (segment (start 155.15 74) (end 149 67.85) (width 0.3) (layer "F.Cu") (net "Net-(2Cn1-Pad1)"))
 (segment (start 106.3 80.65) (end 105.15 79.5) (width 0.3) (layer "F.Cu") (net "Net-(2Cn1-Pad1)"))
 (segment (start 136.926346 67.85) (end 124.126346 80.65) (width 0.3) (layer "F.Cu") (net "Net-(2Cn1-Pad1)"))
 (segment (start 155 73.85) (end 155.15 74) (width 0.3) (layer "F.Cu") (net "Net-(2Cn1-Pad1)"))
 (segment (start 149 67.85) (end 136.926346 67.85) (width 0.3) (layer "F.Cu") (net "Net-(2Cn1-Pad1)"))
 (segment (start 155 67.75) (end 155 73.85) (width 0.3) (layer "F.Cu") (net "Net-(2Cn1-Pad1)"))
 (segment (start 124.126346 80.65) (end 106.3 80.65) (width 0.3) (layer "F.Cu") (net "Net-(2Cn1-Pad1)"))
 (segment (start 124.58 105.805) (end 129.025 110.25) (width 0.3) (layer "F.Cu") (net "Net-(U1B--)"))
 (segment (start 129.025 110.25) (end 132.5 110.25) (width 0.3) (layer "F.Cu") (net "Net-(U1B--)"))
 (segment (start 194.5 101.35) (end 194.5 106.08) (width 0.3) (layer "F.Cu") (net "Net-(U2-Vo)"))
 (segment (start 194.5 106.08) (end 193.08 107.5) (width 0.3) (layer "F.Cu") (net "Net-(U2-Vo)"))
 (segment (start 178 90.5) (end 176.5 89) (width 0.3) (layer "F.Cu") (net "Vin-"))
 (segment (start 176.5 89) (end 172.5 89) (width 0.3) (layer "F.Cu") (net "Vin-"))
 (segment (start 171 90.5) (end 171 98.65) (width 0.3) (layer "F.Cu") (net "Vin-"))
 (segment (start 172.5 89) (end 171 90.5) (width 0.3) (layer "F.Cu") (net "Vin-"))
 (segment (start 190.54 116.5) (end 178 103.96) (width 0.3) (layer "F.Cu") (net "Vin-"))
 (segment (start 171 98.65) (end 173 100.65) (width 0.3) (layer "F.Cu") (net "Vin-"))
 (segment (start 146 104.65) (end 128.275 104.65) (width 0.3) (layer "F.Cu") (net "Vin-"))
 (segment (start 128.275 104.65) (end 127.12 105.805) (width 0.3) (layer "F.Cu") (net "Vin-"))
 (segment (start 178 103.96) (end 178 90.5) (width 0.3) (layer "F.Cu") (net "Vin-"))
 (segment (start 181 119.5) (end 176.5 115) (width 0.3) (layer "F.Cu") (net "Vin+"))
 (segment (start 111.725 105.65) (end 111.88 105.805) (width 0.3) (layer "F.Cu") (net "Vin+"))
 (segment (start 189.85 119.5) (end 192.85 116.5) (width 0.3) (layer "F.Cu") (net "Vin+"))
 (segment (start 171.5 115) (end 169.5 113) (width 0.3) (layer "F.Cu") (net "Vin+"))
 (segment (start 101.5 119.5) (end 101.5 107) (width 0.3) (layer "F.Cu") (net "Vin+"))
 (segment (start 169.5 113) (end 153.5 113) (width 0.3) (layer "F.Cu") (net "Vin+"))
 (segment (start 192.85 116.5) (end 193.08 116.5) (width 0.3) (layer "F.Cu") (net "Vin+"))
 (segment (start 176.5 115) (end 171.5 115) (width 0.3) (layer "F.Cu") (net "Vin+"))
 (segment (start 102.85 105.65) (end 105 105.65) (width 0.3) (layer "F.Cu") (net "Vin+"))
 (segment (start 101.5 107) (end 102.85 105.65) (width 0.3) (layer "F.Cu") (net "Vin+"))
 (segment (start 149 117.5) (end 149 125) (width 0.3) (layer "F.Cu") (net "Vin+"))
 (segment (start 189.85 119.5) (end 181 119.5) (width 0.3) (layer "F.Cu") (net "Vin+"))
 (segment (start 149 125) (end 148 126) (width 0.3) (layer "F.Cu") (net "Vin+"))
 (segment (start 105 105.65) (end 111.725 105.65) (width 0.3) (layer "F.Cu") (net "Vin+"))
 (segment (start 153.5 113) (end 149 117.5) (width 0.3) (layer "F.Cu") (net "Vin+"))
 (segment (start 108 126) (end 101.5 119.5) (width 0.3) (layer "F.Cu") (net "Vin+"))
 (segment (start 148 126) (end 108 126) (width 0.3) (layer "F.Cu") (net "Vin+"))
 (segment (start 103 87.75) (end 104.5 89.25) (width 0.3) (layer "F.Cu") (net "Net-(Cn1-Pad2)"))
 (segment (start 124 88.75) (end 105 88.75) (width 0.3) (layer "F.Cu") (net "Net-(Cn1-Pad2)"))
 (segment (start 105 88.75) (end 104.5 89.25) (width 0.3) (layer "F.Cu") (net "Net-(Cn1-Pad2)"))
 (segment (start 105.15 68) (end 103 70.15) (width 0.3) (layer "F.Cu") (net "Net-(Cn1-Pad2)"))
 (segment (start 103 70.15) (end 103 87.75) (width 0.3) (layer "F.Cu") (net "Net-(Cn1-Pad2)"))
 (segment (start 112.1 118.35) (end 112.25 118.5) (width 0.3) (layer "F.Cu") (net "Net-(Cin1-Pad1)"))
 (segment (start 105 118.35) (end 112.1 118.35) (width 0.3) (layer "F.Cu") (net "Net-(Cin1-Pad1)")))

